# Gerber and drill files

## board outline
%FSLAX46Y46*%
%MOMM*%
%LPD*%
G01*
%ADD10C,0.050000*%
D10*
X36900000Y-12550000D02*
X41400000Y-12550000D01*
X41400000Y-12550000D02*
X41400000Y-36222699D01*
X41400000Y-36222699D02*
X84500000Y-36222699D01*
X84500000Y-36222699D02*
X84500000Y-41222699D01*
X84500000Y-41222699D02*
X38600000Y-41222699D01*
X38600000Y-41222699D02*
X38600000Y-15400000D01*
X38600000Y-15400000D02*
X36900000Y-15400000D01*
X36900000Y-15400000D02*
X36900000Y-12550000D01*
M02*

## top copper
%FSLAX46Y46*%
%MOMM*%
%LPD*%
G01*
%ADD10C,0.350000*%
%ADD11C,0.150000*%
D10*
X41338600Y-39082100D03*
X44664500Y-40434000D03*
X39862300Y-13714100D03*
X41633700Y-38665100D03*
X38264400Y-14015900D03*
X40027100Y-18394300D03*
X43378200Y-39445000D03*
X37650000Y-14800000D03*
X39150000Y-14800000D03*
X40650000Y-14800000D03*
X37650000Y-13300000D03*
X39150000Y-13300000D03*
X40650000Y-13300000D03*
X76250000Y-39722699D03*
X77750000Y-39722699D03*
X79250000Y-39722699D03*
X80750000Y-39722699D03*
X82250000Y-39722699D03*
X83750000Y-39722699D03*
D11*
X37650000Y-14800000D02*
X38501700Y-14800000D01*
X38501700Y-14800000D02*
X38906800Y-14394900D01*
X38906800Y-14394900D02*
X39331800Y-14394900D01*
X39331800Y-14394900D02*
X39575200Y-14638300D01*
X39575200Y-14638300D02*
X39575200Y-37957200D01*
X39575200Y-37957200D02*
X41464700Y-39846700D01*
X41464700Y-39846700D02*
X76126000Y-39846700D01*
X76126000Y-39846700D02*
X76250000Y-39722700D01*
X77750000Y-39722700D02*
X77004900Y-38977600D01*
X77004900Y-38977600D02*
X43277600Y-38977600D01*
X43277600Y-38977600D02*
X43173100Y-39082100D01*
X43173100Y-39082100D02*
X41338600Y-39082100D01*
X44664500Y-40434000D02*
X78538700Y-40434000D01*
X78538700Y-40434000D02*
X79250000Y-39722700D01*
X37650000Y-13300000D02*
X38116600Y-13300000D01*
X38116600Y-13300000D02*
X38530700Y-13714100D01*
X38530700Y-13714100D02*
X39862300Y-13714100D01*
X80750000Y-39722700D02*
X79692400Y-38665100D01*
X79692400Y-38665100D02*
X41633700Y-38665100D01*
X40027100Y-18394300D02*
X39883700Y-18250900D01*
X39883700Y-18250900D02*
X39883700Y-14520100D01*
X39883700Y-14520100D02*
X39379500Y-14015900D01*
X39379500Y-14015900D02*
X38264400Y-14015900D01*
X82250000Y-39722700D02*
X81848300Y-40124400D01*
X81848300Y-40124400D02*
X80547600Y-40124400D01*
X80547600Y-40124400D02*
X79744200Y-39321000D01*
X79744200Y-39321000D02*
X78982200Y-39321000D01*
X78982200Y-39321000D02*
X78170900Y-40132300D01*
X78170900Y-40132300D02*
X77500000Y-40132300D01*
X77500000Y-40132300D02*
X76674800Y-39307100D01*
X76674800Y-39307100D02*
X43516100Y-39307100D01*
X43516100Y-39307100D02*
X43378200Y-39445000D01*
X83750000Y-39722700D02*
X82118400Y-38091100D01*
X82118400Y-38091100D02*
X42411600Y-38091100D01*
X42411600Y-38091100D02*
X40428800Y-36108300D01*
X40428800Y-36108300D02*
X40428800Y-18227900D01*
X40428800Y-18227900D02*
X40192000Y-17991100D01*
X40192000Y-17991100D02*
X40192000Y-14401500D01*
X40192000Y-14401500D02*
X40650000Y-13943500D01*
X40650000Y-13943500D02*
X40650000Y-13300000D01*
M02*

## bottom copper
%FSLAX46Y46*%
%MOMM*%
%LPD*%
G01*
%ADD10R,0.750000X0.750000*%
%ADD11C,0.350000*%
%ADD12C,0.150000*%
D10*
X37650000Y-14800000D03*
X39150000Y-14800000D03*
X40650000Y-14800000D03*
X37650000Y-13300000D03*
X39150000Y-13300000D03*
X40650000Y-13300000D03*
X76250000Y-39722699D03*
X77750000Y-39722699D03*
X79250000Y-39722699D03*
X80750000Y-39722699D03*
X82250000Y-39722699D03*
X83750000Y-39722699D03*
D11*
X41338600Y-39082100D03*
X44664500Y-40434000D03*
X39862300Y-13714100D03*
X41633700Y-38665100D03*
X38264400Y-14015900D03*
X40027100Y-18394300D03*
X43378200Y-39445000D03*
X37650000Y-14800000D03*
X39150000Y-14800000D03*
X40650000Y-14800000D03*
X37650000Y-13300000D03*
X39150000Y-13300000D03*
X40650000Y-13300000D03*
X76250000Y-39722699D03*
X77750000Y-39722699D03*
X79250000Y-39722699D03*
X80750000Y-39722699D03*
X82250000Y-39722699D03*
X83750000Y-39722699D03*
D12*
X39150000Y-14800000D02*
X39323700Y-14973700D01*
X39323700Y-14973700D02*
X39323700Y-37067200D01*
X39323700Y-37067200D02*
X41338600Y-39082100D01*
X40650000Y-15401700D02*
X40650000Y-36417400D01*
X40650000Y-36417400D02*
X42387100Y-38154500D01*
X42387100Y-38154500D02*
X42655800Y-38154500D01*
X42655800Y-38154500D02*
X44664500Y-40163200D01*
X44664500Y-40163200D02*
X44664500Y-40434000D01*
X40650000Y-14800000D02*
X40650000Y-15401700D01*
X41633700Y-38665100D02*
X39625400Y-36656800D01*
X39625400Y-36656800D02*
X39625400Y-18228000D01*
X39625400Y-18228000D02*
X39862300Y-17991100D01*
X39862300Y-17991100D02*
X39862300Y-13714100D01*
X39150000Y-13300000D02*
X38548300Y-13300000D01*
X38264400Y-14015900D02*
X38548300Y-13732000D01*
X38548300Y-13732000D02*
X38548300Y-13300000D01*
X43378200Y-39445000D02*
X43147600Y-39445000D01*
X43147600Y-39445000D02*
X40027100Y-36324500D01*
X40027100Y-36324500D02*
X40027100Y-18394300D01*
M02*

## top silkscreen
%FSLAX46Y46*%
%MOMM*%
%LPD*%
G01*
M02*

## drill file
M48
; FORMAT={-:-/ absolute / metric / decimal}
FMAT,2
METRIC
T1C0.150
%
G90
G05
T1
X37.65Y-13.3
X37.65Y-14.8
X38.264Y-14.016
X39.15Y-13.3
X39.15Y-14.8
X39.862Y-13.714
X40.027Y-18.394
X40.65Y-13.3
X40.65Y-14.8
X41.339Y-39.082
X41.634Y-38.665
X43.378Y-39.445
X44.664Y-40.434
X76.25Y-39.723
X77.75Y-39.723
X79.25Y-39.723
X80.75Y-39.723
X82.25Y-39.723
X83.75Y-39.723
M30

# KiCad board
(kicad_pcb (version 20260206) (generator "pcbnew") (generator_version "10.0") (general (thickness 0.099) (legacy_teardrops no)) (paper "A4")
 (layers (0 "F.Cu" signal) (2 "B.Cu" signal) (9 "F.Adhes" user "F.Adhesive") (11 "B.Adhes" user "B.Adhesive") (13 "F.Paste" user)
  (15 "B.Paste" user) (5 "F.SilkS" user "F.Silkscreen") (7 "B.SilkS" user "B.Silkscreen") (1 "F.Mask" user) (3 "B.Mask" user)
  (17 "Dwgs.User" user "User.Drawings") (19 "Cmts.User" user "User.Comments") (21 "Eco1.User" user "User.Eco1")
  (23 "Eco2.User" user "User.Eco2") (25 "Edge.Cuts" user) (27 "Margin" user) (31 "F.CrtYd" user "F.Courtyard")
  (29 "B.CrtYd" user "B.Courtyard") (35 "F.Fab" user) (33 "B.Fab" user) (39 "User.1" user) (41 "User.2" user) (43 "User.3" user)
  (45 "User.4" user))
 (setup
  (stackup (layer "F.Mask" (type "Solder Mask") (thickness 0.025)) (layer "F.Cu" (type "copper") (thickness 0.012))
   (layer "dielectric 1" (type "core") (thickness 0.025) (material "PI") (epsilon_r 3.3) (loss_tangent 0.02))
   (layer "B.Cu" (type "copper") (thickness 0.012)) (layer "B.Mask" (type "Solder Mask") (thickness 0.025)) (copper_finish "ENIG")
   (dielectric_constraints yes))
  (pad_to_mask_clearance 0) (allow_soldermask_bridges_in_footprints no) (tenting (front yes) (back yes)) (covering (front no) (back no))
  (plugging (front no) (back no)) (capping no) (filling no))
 (gr_line (start 36.900000000000006 12.55) (end 41.400000000000006 12.55) (stroke (width 0.05) (type default)) (layer "Edge.Cuts"))
 (gr_line (start 41.400000000000006 12.55) (end 41.4 36.22269878025519) (stroke (width 0.05) (type default)) (layer "Edge.Cuts"))
 (gr_line (start 41.4 36.22269878025519) (end 84.5 36.22269878025519) (stroke (width 0.05) (type default)) (layer "Edge.Cuts"))
 (gr_line (start 84.5 36.22269878025519) (end 84.5 41.22269878025519) (stroke (width 0.05) (type default)) (layer "Edge.Cuts"))
 (gr_line (start 84.5 41.22269878025519) (end 38.6 41.22269878025519) (stroke (width 0.05) (type default)) (layer "Edge.Cuts"))
 (gr_line (start 38.6 41.22269878025519) (end 38.6 15.4) (stroke (width 0.05) (type default)) (layer "Edge.Cuts"))
 (gr_line (start 38.6 15.4) (end 36.900000000000006 15.4) (stroke (width 0.05) (type default)) (layer "Edge.Cuts"))
 (gr_line (start 36.900000000000006 15.4) (end 36.900000000000006 12.55) (stroke (width 0.05) (type default)) (layer "Edge.Cuts"))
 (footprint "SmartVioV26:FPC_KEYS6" (layer "F.Cu") (at 0 0)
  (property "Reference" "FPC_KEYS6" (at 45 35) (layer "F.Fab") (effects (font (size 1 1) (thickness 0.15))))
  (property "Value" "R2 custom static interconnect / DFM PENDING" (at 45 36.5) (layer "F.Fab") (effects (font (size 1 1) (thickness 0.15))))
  (pad "S1" smd rect (at 37.650000000000006 14.8) (size 0.75 0.75) (layers "B.Cu" "B.Mask") (solder_mask_margin 0.1) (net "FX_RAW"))
  (pad "S2" smd rect (at 39.150000000000006 14.8) (size 0.75 0.75) (layers "B.Cu" "B.Mask") (solder_mask_margin 0.1) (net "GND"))
  (pad "S3" smd rect (at 40.650000000000006 14.8) (size 0.75 0.75) (layers "B.Cu" "B.Mask") (solder_mask_margin 0.1) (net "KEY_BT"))
  (pad "S4" smd rect (at 37.650000000000006 13.3) (size 0.75 0.75) (layers "B.Cu" "B.Mask") (solder_mask_margin 0.1) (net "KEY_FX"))
  (pad "S5" smd rect (at 39.150000000000006 13.3) (size 0.75 0.75) (layers "B.Cu" "B.Mask") (solder_mask_margin 0.1) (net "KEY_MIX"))
  (pad "S6" smd rect (at 40.650000000000006 13.3) (size 0.75 0.75) (layers "B.Cu" "B.Mask") (solder_mask_margin 0.1) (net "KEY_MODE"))
  (pad "T1" smd rect (at 76.25 39.72269878025519) (size 0.75 0.75) (layers "B.Cu" "B.Mask") (solder_mask_margin 0.1) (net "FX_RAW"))
  (pad "T2" smd rect (at 77.75 39.72269878025519) (size 0.75 0.75) (layers "B.Cu" "B.Mask") (solder_mask_margin 0.1) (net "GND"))
  (pad "T3" smd rect (at 79.25 39.72269878025519) (size 0.75 0.75) (layers "B.Cu" "B.Mask") (solder_mask_margin 0.1) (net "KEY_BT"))
  (pad "T4" smd rect (at 80.75 39.72269878025519) (size 0.75 0.75) (layers "B.Cu" "B.Mask") (solder_mask_margin 0.1) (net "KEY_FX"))
  (pad "T5" smd rect (at 82.25 39.72269878025519) (size 0.75 0.75) (layers "B.Cu" "B.Mask") (solder_mask_margin 0.1) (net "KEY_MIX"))
  (pad "T6" smd rect (at 83.75 39.72269878025519) (size 0.75 0.75) (layers "B.Cu" "B.Mask") (solder_mask_margin 0.1) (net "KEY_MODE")))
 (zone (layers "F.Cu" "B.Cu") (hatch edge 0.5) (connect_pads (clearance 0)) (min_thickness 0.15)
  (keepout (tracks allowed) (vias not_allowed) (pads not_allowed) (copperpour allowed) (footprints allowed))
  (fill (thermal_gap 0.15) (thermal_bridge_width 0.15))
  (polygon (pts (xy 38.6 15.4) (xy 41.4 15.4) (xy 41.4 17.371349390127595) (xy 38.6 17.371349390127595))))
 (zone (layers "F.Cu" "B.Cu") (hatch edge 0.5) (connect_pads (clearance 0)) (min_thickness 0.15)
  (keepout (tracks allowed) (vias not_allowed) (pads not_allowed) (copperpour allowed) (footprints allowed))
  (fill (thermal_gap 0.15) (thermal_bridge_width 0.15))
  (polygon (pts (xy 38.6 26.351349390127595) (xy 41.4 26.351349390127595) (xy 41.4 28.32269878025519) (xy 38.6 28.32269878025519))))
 (segment (start 37.65 14.8) (end 38.5017 14.8) (width 0.15) (layer "F.Cu") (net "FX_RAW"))
 (segment (start 38.5017 14.8) (end 38.9068 14.3949) (width 0.15) (layer "F.Cu") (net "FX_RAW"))
 (segment (start 38.9068 14.3949) (end 39.3318 14.3949) (width 0.15) (layer "F.Cu") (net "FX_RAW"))
 (segment (start 39.3318 14.3949) (end 39.5752 14.6383) (width 0.15) (layer "F.Cu") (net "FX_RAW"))
 (segment (start 39.5752 14.6383) (end 39.5752 37.9572) (width 0.15) (layer "F.Cu") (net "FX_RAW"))
 (segment (start 39.5752 37.9572) (end 41.4647 39.8467) (width 0.15) (layer "F.Cu") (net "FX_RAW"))
 (segment (start 41.4647 39.8467) (end 76.126 39.8467) (width 0.15) (layer "F.Cu") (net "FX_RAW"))
 (segment (start 76.126 39.8467) (end 76.25 39.7227) (width 0.15) (layer "F.Cu") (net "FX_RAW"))
 (segment (start 39.15 14.8) (end 39.3237 14.9737) (width 0.15) (layer "B.Cu") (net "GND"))
 (segment (start 39.3237 14.9737) (end 39.3237 37.0672) (width 0.15) (layer "B.Cu") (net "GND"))
 (segment (start 39.3237 37.0672) (end 41.3386 39.0821) (width 0.15) (layer "B.Cu") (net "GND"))
 (segment (start 77.75 39.7227) (end 77.0049 38.9776) (width 0.15) (layer "F.Cu") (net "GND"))
 (segment (start 77.0049 38.9776) (end 43.2776 38.9776) (width 0.15) (layer "F.Cu") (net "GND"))
 (segment (start 43.2776 38.9776) (end 43.1731 39.0821) (width 0.15) (layer "F.Cu") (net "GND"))
 (segment (start 43.1731 39.0821) (end 41.3386 39.0821) (width 0.15) (layer "F.Cu") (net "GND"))
 (via (at 41.3386 39.0821) (size 0.35) (drill 0.15) (layers "F.Cu" "B.Cu") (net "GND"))
 (segment (start 44.6645 40.434) (end 78.5387 40.434) (width 0.15) (layer "F.Cu") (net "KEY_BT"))
 (segment (start 78.5387 40.434) (end 79.25 39.7227) (width 0.15) (layer "F.Cu") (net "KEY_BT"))
 (segment (start 40.65 15.4017) (end 40.65 36.4174) (width 0.15) (layer "B.Cu") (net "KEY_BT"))
 (segment (start 40.65 36.4174) (end 42.3871 38.1545) (width 0.15) (layer "B.Cu") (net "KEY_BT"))
 (segment (start 42.3871 38.1545) (end 42.6558 38.1545) (width 0.15) (layer "B.Cu") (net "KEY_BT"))
 (segment (start 42.6558 38.1545) (end 44.6645 40.1632) (width 0.15) (layer "B.Cu") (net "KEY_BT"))
 (segment (start 44.6645 40.1632) (end 44.6645 40.434) (width 0.15) (layer "B.Cu") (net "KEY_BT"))
 (segment (start 40.65 14.8) (end 40.65 15.4017) (width 0.15) (layer "B.Cu") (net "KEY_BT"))
 (via (at 44.6645 40.434) (size 0.35) (drill 0.15) (layers "F.Cu" "B.Cu") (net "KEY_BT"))
 (segment (start 37.65 13.3) (end 38.1166 13.3) (width 0.15) (layer "F.Cu") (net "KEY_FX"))
 (segment (start 38.1166 13.3) (end 38.5307 13.7141) (width 0.15) (layer "F.Cu") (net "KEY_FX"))
 (segment (start 38.5307 13.7141) (end 39.8623 13.7141) (width 0.15) (layer "F.Cu") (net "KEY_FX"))
 (segment (start 41.6337 38.6651) (end 39.6254 36.6568) (width 0.15) (layer "B.Cu") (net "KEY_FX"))
 (segment (start 39.6254 36.6568) (end 39.6254 18.228) (width 0.15) (layer "B.Cu") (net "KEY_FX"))
 (segment (start 39.6254 18.228) (end 39.8623 17.9911) (width 0.15) (layer "B.Cu") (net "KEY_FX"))
 (segment (start 39.8623 17.9911) (end 39.8623 13.7141) (width 0.15) (layer "B.Cu") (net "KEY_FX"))
 (segment (start 80.75 39.7227) (end 79.6924 38.6651) (width 0.15) (layer "F.Cu") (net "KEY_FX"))
 (segment (start 79.6924 38.6651) (end 41.6337 38.6651) (width 0.15) (layer "F.Cu") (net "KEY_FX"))
 (via (at 39.8623 13.7141) (size 0.35) (drill 0.15) (layers "F.Cu" "B.Cu") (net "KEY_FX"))
 (via (at 41.6337 38.6651) (size 0.35) (drill 0.15) (layers "F.Cu" "B.Cu") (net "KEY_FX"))
 (segment (start 39.15 13.3) (end 38.5483 13.3) (width 0.15) (layer "B.Cu") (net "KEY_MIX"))
 (segment (start 38.2644 14.0159) (end 38.5483 13.732) (width 0.15) (layer "B.Cu") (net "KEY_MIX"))
 (segment (start 38.5483 13.732) (end 38.5483 13.3) (width 0.15) (layer "B.Cu") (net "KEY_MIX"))
 (via (at 38.2644 14.0159) (size 0.35) (drill 0.15) (layers "F.Cu" "B.Cu") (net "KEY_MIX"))
 (segment (start 40.0271 18.3943) (end 39.8837 18.2509) (width 0.15) (layer "F.Cu") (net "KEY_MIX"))
 (segment (start 39.8837 18.2509) (end 39.8837 14.5201) (width 0.15) (layer "F.Cu") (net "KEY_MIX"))
 (segment (start 39.8837 14.5201) (end 39.3795 14.0159) (width 0.15) (layer "F.Cu") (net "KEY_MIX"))
 (segment (start 39.3795 14.0159) (end 38.2644 14.0159) (width 0.15) (layer "F.Cu") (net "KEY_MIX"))
 (via (at 40.0271 18.3943) (size 0.35) (drill 0.15) (layers "F.Cu" "B.Cu") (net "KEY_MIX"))
 (segment (start 43.3782 39.445) (end 43.1476 39.445) (width 0.15) (layer "B.Cu") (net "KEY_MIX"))
 (segment (start 43.1476 39.445) (end 40.0271 36.3245) (width 0.15) (layer "B.Cu") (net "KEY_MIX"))
 (segment (start 40.0271 36.3245) (end 40.0271 18.3943) (width 0.15) (layer "B.Cu") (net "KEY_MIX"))
 (via (at 43.3782 39.445) (size 0.35) (drill 0.15) (layers "F.Cu" "B.Cu") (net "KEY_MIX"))
 (segment (start 82.25 39.7227) (end 81.8483 40.1244) (width 0.15) (layer "F.Cu") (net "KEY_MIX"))
 (segment (start 81.8483 40.1244) (end 80.5476 40.1244) (width 0.15) (layer "F.Cu") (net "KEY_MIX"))
 (segment (start 80.5476 40.1244) (end 79.7442 39.321) (width 0.15) (layer "F.Cu") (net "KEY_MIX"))
 (segment (start 79.7442 39.321) (end 78.9822 39.321) (width 0.15) (layer "F.Cu") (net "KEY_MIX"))
 (segment (start 78.9822 39.321) (end 78.1709 40.1323) (width 0.15) (layer "F.Cu") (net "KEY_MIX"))
 (segment (start 78.1709 40.1323) (end 77.5 40.1323) (width 0.15) (layer "F.Cu") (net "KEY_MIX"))
 (segment (start 77.5 40.1323) (end 76.6748 39.3071) (width 0.15) (layer "F.Cu") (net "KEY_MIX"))
 (segment (start 76.6748 39.3071) (end 43.5161 39.3071) (width 0.15) (layer "F.Cu") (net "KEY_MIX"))
 (segment (start 43.5161 39.3071) (end 43.3782 39.445) (width 0.15) (layer "F.Cu") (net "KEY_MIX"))
 (segment (start 83.75 39.7227) (end 82.1184 38.0911) (width 0.15) (layer "F.Cu") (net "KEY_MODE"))
 (segment (start 82.1184 38.0911) (end 42.4116 38.0911) (width 0.15) (layer "F.Cu") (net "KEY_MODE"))
 (segment (start 42.4116 38.0911) (end 40.4288 36.1083) (width 0.15) (layer "F.Cu") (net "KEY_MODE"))
 (segment (start 40.4288 36.1083) (end 40.4288 18.2279) (width 0.15) (layer "F.Cu") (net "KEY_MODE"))
 (segment (start 40.4288 18.2279) (end 40.192 17.9911) (width 0.15) (layer "F.Cu") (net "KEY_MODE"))
 (segment (start 40.192 17.9911) (end 40.192 14.4015) (width 0.15) (layer "F.Cu") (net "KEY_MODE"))
 (segment (start 40.192 14.4015) (end 40.65 13.9435) (width 0.15) (layer "F.Cu") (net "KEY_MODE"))
 (segment (start 40.65 13.9435) (end 40.65 13.3) (width 0.15) (layer "F.Cu") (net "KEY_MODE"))
 (via (at 37.650000000000006 14.8) (size 0.35) (drill 0.15) (layers "F.Cu" "B.Cu") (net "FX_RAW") (locked yes))
 (via (at 39.150000000000006 14.8) (size 0.35) (drill 0.15) (layers "F.Cu" "B.Cu") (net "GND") (locked yes))
 (via (at 40.650000000000006 14.8) (size 0.35) (drill 0.15) (layers "F.Cu" "B.Cu") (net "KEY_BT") (locked yes))
 (via (at 37.650000000000006 13.3) (size 0.35) (drill 0.15) (layers "F.Cu" "B.Cu") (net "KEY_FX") (locked yes))
 (via (at 39.150000000000006 13.3) (size 0.35) (drill 0.15) (layers "F.Cu" "B.Cu") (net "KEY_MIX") (locked yes))
 (via (at 40.650000000000006 13.3) (size 0.35) (drill 0.15) (layers "F.Cu" "B.Cu") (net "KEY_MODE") (locked yes))
 (via (at 76.25 39.72269878025519) (size 0.35) (drill 0.15) (layers "F.Cu" "B.Cu") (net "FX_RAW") (locked yes))
 (via (at 77.75 39.72269878025519) (size 0.35) (drill 0.15) (layers "F.Cu" "B.Cu") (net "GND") (locked yes))
 (via (at 79.25 39.72269878025519) (size 0.35) (drill 0.15) (layers "F.Cu" "B.Cu") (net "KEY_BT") (locked yes))
 (via (at 80.75 39.72269878025519) (size 0.35) (drill 0.15) (layers "F.Cu" "B.Cu") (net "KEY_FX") (locked yes))
 (via (at 82.25 39.72269878025519) (size 0.35) (drill 0.15) (layers "F.Cu" "B.Cu") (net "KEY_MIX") (locked yes))
 (via (at 83.75 39.72269878025519) (size 0.35) (drill 0.15) (layers "F.Cu" "B.Cu") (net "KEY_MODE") (locked yes)))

